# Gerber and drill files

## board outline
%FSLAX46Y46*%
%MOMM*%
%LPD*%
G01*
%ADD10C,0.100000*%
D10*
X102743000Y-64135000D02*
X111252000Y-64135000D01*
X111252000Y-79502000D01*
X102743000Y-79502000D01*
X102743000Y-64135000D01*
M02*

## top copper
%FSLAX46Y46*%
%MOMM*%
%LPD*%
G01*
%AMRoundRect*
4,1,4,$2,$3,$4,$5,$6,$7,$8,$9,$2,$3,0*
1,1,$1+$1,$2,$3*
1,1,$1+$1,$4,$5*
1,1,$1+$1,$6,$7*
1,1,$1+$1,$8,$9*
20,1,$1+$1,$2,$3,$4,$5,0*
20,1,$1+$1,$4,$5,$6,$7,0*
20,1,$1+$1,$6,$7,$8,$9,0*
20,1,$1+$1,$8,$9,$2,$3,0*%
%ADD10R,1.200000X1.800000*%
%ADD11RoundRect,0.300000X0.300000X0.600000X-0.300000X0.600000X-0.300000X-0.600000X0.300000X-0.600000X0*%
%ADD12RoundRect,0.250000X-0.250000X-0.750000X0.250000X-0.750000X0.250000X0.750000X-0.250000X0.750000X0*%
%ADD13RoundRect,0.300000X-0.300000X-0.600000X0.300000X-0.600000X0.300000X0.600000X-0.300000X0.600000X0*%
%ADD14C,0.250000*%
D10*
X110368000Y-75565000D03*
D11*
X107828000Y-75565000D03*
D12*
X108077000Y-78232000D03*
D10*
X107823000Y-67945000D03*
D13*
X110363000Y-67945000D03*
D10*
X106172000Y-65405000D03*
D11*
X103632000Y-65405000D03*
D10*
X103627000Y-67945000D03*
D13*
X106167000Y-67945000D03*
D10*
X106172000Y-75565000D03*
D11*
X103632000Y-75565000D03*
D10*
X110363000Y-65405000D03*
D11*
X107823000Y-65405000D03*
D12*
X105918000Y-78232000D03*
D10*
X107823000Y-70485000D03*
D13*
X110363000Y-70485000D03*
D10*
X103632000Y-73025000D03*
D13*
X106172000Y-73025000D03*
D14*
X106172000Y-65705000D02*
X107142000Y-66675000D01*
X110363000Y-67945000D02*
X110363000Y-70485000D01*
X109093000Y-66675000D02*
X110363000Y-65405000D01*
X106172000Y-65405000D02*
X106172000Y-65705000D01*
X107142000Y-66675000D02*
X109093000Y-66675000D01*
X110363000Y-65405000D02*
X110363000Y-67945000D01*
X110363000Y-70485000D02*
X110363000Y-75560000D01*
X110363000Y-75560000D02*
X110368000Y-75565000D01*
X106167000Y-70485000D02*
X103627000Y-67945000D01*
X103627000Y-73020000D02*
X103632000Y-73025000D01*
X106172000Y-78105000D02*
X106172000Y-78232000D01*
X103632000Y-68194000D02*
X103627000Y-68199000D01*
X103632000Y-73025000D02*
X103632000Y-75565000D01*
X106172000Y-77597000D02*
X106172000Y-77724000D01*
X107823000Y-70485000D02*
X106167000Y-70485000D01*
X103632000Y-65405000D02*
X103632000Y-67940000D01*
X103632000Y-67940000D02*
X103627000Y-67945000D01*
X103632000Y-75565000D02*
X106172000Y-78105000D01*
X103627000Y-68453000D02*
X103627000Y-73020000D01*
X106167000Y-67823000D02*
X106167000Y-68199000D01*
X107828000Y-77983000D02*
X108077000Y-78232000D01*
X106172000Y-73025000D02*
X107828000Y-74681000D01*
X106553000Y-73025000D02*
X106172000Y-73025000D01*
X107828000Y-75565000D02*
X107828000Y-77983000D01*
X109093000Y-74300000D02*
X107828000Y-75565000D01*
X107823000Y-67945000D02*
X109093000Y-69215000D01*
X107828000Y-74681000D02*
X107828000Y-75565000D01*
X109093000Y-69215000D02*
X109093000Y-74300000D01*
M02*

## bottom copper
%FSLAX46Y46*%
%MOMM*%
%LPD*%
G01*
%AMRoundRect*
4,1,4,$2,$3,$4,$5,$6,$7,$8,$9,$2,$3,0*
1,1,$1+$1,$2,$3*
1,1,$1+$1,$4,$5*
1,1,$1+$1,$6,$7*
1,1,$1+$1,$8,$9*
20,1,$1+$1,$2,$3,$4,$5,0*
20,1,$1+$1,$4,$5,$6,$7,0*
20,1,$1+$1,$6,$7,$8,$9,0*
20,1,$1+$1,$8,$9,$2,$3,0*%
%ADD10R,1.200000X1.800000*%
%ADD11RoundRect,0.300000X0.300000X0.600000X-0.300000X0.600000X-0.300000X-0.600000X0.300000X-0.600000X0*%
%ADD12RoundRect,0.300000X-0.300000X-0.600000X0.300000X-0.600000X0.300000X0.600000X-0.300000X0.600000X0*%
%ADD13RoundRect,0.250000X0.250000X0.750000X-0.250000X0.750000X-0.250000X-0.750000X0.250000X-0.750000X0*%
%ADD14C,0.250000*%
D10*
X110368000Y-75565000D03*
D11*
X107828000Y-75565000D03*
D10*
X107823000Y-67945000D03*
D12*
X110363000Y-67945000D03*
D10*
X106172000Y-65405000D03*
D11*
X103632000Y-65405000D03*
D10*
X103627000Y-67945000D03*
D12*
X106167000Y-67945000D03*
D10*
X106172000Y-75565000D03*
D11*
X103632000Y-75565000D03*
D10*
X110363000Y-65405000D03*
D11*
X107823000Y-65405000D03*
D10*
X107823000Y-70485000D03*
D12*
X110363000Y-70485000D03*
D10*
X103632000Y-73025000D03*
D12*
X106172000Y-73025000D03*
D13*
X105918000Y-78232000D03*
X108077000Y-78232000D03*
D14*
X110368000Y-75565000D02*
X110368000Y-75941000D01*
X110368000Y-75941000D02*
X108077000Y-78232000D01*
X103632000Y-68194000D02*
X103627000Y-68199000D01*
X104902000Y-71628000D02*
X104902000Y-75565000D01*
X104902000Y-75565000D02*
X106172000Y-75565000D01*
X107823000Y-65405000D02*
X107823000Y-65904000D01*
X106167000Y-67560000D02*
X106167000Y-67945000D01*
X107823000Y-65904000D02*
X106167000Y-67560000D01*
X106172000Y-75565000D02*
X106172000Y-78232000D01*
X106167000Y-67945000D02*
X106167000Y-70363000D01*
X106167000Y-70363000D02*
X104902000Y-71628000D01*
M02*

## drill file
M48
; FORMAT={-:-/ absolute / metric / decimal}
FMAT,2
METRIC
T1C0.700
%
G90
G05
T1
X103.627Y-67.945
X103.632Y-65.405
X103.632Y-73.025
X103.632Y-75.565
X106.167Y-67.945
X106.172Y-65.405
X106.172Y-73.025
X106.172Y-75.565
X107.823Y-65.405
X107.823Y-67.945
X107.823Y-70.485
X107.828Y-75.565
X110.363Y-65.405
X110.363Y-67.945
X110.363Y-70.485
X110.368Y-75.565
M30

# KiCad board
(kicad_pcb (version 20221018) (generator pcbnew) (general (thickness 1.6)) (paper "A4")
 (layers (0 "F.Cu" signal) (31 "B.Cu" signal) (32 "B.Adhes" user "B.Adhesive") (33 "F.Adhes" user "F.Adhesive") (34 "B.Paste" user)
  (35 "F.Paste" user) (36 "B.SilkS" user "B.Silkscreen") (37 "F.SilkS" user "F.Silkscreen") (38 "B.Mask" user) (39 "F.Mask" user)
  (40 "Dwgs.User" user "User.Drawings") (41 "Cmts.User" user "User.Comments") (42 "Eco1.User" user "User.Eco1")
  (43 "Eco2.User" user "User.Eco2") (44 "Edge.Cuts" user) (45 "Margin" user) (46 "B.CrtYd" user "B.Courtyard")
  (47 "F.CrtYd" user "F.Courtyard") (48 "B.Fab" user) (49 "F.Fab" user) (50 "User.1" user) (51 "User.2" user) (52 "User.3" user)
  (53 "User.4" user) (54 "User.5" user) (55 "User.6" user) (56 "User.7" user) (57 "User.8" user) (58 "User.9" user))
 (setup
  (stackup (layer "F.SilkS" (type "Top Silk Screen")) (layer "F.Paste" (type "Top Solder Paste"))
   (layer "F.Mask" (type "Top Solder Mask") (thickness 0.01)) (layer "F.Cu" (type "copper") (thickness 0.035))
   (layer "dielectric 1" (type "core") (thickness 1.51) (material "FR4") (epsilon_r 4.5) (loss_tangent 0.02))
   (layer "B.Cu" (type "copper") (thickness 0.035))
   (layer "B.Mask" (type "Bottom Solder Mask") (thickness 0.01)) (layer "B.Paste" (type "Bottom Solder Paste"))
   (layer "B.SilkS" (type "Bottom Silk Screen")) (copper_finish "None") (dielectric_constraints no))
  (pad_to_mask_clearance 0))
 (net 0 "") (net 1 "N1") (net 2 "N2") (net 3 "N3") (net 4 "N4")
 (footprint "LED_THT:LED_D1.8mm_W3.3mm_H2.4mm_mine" (layer "F.Cu") (at 110.368 75.565 180)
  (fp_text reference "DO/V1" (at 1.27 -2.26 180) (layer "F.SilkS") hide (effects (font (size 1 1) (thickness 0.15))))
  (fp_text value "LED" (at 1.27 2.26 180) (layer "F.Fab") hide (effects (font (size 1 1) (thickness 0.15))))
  (pad "1" thru_hole rect (at 0 0 180) (size 1.2 1.8) (drill 0.7) (layers "*.Cu" "*.Mask") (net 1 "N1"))
  (pad "2" thru_hole roundrect (at 2.54 0 180) (size 1.2 1.8) (drill 0.7) (layers "*.Cu" "*.Mask") (roundrect_rratio 0.25) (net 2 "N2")))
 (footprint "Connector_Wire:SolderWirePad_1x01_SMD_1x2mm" (layer "F.Cu") (at 108.077 78.232)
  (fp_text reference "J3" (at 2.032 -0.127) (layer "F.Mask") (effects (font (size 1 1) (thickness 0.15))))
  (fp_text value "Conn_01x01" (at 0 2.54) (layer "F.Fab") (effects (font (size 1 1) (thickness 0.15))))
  (pad "1" smd roundrect (at 0 0) (size 1 2) (layers "F.Cu" "F.Paste" "F.Mask") (roundrect_rratio 0.25) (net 2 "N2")))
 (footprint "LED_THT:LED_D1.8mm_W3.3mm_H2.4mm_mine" (layer "F.Cu") (at 107.823 67.945)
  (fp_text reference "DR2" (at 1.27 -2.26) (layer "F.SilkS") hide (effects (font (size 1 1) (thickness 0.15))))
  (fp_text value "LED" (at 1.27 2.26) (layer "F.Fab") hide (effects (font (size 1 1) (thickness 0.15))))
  (pad "1" thru_hole rect (at 0 0) (size 1.2 1.8) (drill 0.7) (layers "*.Cu" "*.Mask") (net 2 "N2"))
  (pad "2" thru_hole roundrect (at 2.54 0) (size 1.2 1.8) (drill 0.7) (layers "*.Cu" "*.Mask") (roundrect_rratio 0.25) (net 1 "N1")))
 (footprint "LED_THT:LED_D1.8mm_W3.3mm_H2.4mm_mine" (layer "F.Cu") (at 106.172 65.405 180)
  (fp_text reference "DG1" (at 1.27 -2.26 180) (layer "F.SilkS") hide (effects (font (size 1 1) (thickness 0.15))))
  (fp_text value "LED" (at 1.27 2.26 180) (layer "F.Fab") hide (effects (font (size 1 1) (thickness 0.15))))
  (pad "1" thru_hole rect (at 0 0 180) (size 1.2 1.8) (drill 0.7) (layers "*.Cu" "*.Mask") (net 1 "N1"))
  (pad "2" thru_hole roundrect (at 2.54 0 180) (size 1.2 1.8) (drill 0.7) (layers "*.Cu" "*.Mask") (roundrect_rratio 0.25) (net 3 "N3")))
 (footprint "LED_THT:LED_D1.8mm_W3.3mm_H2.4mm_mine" (layer "F.Cu") (at 103.627 67.945)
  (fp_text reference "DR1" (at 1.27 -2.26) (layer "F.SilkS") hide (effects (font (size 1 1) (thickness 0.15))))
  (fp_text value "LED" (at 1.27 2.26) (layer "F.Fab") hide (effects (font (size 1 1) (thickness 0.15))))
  (pad "1" thru_hole rect (at 0 0) (size 1.2 1.8) (drill 0.7) (layers "*.Cu" "*.Mask") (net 3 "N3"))
  (pad "2" thru_hole roundrect (at 2.54 0) (size 1.2 1.8) (drill 0.7) (layers "*.Cu" "*.Mask") (roundrect_rratio 0.25) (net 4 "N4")))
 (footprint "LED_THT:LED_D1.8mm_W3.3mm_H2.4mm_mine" (layer "F.Cu") (at 106.172 75.565 180)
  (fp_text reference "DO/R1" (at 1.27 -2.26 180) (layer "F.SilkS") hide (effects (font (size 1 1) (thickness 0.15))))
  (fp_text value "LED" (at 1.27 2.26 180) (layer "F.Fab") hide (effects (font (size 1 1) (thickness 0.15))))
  (pad "1" thru_hole rect (at 0 0 180) (size 1.2 1.8) (drill 0.7) (layers "*.Cu" "*.Mask") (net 4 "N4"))
  (pad "2" thru_hole roundrect (at 2.54 0 180) (size 1.2 1.8) (drill 0.7) (layers "*.Cu" "*.Mask") (roundrect_rratio 0.25) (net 3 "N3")))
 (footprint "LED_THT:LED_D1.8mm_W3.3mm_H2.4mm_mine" (layer "F.Cu") (at 110.363 65.405 180)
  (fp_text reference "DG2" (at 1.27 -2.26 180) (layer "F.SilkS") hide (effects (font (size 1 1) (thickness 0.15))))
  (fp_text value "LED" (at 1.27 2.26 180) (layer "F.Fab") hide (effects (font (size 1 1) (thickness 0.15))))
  (pad "1" thru_hole rect (at 0 0 180) (size 1.2 1.8) (drill 0.7) (layers "*.Cu" "*.Mask") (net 1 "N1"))
  (pad "2" thru_hole roundrect (at 2.54 0 180) (size 1.2 1.8) (drill 0.7) (layers "*.Cu" "*.Mask") (roundrect_rratio 0.25) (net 4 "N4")))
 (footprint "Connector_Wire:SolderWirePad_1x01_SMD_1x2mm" (layer "F.Cu") (at 105.918 78.232)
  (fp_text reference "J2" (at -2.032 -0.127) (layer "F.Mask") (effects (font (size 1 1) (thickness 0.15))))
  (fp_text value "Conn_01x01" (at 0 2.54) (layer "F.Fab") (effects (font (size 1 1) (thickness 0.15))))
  (pad "1" smd roundrect (at 0 0) (size 1 2) (layers "F.Cu" "F.Paste" "F.Mask") (roundrect_rratio 0.25) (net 3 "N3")))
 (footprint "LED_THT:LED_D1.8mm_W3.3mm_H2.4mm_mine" (layer "F.Cu") (at 107.823 70.485)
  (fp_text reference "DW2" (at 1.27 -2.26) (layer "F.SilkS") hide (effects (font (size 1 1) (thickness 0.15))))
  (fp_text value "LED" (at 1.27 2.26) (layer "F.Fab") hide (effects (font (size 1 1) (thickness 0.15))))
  (pad "1" thru_hole rect (at 0 0) (size 1.2 1.8) (drill 0.7) (layers "*.Cu" "*.Mask") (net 3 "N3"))
  (pad "2" thru_hole roundrect (at 2.54 0) (size 1.2 1.8) (drill 0.7) (layers "*.Cu" "*.Mask") (roundrect_rratio 0.25) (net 1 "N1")))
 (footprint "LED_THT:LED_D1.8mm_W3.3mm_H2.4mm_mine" (layer "F.Cu") (at 103.632 73.025)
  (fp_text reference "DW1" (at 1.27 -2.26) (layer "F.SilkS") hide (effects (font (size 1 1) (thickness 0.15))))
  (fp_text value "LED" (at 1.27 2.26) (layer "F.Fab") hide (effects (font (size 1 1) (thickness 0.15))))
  (pad "1" thru_hole rect (at 0 0) (size 1.2 1.8) (drill 0.7) (layers "*.Cu" "*.Mask") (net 3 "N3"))
  (pad "2" thru_hole roundrect (at 2.54 0) (size 1.2 1.8) (drill 0.7) (layers "*.Cu" "*.Mask") (roundrect_rratio 0.25) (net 2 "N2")))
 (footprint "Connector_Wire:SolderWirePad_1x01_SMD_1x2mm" (layer "B.Cu") (at 105.918 78.232 180)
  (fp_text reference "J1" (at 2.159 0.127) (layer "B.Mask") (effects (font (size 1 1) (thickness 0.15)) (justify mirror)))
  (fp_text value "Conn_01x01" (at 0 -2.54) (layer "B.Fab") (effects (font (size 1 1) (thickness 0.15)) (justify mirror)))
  (pad "1" smd roundrect (at 0 0 180) (size 1 2) (layers "B.Cu" "B.Paste" "B.Mask") (roundrect_rratio 0.25) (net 4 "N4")))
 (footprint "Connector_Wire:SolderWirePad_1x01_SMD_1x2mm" (layer "B.Cu") (at 108.077 78.232 180)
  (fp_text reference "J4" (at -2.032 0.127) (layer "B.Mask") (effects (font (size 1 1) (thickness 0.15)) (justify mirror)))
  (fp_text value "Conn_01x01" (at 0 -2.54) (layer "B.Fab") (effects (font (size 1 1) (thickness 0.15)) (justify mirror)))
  (pad "1" smd roundrect (at 0 0 180) (size 1 2) (layers "B.Cu" "B.Paste" "B.Mask") (roundrect_rratio 0.25) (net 1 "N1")))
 (gr_rect (start 102.743 64.135) (end 111.252 79.502) (stroke (width 0.1) (type default)) (fill none) (layer "Edge.Cuts"))
 (segment (start 106.172 65.705) (end 107.142 66.675) (width 0.25) (layer "F.Cu") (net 1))
 (segment (start 110.363 67.945) (end 110.363 70.485) (width 0.25) (layer "F.Cu") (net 1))
 (segment (start 109.093 66.675) (end 110.363 65.405) (width 0.25) (layer "F.Cu") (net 1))
 (segment (start 106.172 65.405) (end 106.172 65.705) (width 0.25) (layer "F.Cu") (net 1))
 (segment (start 107.142 66.675) (end 109.093 66.675) (width 0.25) (layer "F.Cu") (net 1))
 (segment (start 110.363 65.405) (end 110.363 67.945) (width 0.25) (layer "F.Cu") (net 1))
 (segment (start 110.363 70.485) (end 110.363 75.56) (width 0.25) (layer "F.Cu") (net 1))
 (segment (start 110.363 75.56) (end 110.368 75.565) (width 0.25) (layer "F.Cu") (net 1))
 (segment (start 110.368 75.565) (end 110.368 75.941) (width 0.25) (layer "B.Cu") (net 1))
 (segment (start 110.368 75.941) (end 108.077 78.232) (width 0.25) (layer "B.Cu") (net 1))
 (segment (start 106.167 70.485) (end 103.627 67.945) (width 0.25) (layer "F.Cu") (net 3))
 (segment (start 103.627 73.02) (end 103.632 73.025) (width 0.25) (layer "F.Cu") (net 3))
 (segment (start 106.172 78.105) (end 106.172 78.232) (width 0.25) (layer "F.Cu") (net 3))
 (segment (start 103.632 68.194) (end 103.627 68.199) (width 0.25) (layer "F.Cu") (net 3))
 (segment (start 103.632 73.025) (end 103.632 75.565) (width 0.25) (layer "F.Cu") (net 3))
 (segment (start 106.172 77.597) (end 106.172 77.724) (width 0.25) (layer "F.Cu") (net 3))
 (segment (start 107.823 70.485) (end 106.167 70.485) (width 0.25) (layer "F.Cu") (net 3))
 (segment (start 103.632 65.405) (end 103.632 67.94) (width 0.25) (layer "F.Cu") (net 3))
 (segment (start 103.632 67.94) (end 103.627 67.945) (width 0.25) (layer "F.Cu") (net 3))
 (segment (start 103.632 75.565) (end 106.172 78.105) (width 0.25) (layer "F.Cu") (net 3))
 (segment (start 103.627 68.453) (end 103.627 73.02) (width 0.25) (layer "F.Cu") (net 3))
 (segment (start 103.632 68.194) (end 103.627 68.199) (width 0.25) (layer "B.Cu") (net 3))
 (segment (start 106.167 67.823) (end 106.167 68.199) (width 0.25) (layer "F.Cu") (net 4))
 (segment (start 104.902 71.628) (end 104.902 75.565) (width 0.25) (layer "B.Cu") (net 4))
 (segment (start 104.902 75.565) (end 106.172 75.565) (width 0.25) (layer "B.Cu") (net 4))
 (segment (start 107.823 65.405) (end 107.823 65.904) (width 0.25) (layer "B.Cu") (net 4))
 (segment (start 106.167 67.56) (end 106.167 67.945) (width 0.25) (layer "B.Cu") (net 4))
 (segment (start 107.823 65.904) (end 106.167 67.56) (width 0.25) (layer "B.Cu") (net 4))
 (segment (start 106.172 75.565) (end 106.172 78.232) (width 0.25) (layer "B.Cu") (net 4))
 (segment (start 106.167 67.945) (end 106.167 70.363) (width 0.25) (layer "B.Cu") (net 4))
 (segment (start 106.167 70.363) (end 104.902 71.628) (width 0.25) (layer "B.Cu") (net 4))
 (segment (start 107.828 77.983) (end 108.077 78.232) (width 0.25) (layer "F.Cu") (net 2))
 (segment (start 106.172 73.025) (end 107.828 74.681) (width 0.25) (layer "F.Cu") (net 2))
 (segment (start 106.553 73.025) (end 106.172 73.025) (width 0.25) (layer "F.Cu") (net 2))
 (segment (start 107.828 75.565) (end 107.828 77.983) (width 0.25) (layer "F.Cu") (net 2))
 (segment (start 109.093 74.3) (end 107.828 75.565) (width 0.25) (layer "F.Cu") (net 2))
 (segment (start 107.823 67.945) (end 109.093 69.215) (width 0.25) (layer "F.Cu") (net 2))
 (segment (start 107.828 74.681) (end 107.828 75.565) (width 0.25) (layer "F.Cu") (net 2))
 (segment (start 109.093 69.215) (end 109.093 74.3) (width 0.25) (layer "F.Cu") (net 2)))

